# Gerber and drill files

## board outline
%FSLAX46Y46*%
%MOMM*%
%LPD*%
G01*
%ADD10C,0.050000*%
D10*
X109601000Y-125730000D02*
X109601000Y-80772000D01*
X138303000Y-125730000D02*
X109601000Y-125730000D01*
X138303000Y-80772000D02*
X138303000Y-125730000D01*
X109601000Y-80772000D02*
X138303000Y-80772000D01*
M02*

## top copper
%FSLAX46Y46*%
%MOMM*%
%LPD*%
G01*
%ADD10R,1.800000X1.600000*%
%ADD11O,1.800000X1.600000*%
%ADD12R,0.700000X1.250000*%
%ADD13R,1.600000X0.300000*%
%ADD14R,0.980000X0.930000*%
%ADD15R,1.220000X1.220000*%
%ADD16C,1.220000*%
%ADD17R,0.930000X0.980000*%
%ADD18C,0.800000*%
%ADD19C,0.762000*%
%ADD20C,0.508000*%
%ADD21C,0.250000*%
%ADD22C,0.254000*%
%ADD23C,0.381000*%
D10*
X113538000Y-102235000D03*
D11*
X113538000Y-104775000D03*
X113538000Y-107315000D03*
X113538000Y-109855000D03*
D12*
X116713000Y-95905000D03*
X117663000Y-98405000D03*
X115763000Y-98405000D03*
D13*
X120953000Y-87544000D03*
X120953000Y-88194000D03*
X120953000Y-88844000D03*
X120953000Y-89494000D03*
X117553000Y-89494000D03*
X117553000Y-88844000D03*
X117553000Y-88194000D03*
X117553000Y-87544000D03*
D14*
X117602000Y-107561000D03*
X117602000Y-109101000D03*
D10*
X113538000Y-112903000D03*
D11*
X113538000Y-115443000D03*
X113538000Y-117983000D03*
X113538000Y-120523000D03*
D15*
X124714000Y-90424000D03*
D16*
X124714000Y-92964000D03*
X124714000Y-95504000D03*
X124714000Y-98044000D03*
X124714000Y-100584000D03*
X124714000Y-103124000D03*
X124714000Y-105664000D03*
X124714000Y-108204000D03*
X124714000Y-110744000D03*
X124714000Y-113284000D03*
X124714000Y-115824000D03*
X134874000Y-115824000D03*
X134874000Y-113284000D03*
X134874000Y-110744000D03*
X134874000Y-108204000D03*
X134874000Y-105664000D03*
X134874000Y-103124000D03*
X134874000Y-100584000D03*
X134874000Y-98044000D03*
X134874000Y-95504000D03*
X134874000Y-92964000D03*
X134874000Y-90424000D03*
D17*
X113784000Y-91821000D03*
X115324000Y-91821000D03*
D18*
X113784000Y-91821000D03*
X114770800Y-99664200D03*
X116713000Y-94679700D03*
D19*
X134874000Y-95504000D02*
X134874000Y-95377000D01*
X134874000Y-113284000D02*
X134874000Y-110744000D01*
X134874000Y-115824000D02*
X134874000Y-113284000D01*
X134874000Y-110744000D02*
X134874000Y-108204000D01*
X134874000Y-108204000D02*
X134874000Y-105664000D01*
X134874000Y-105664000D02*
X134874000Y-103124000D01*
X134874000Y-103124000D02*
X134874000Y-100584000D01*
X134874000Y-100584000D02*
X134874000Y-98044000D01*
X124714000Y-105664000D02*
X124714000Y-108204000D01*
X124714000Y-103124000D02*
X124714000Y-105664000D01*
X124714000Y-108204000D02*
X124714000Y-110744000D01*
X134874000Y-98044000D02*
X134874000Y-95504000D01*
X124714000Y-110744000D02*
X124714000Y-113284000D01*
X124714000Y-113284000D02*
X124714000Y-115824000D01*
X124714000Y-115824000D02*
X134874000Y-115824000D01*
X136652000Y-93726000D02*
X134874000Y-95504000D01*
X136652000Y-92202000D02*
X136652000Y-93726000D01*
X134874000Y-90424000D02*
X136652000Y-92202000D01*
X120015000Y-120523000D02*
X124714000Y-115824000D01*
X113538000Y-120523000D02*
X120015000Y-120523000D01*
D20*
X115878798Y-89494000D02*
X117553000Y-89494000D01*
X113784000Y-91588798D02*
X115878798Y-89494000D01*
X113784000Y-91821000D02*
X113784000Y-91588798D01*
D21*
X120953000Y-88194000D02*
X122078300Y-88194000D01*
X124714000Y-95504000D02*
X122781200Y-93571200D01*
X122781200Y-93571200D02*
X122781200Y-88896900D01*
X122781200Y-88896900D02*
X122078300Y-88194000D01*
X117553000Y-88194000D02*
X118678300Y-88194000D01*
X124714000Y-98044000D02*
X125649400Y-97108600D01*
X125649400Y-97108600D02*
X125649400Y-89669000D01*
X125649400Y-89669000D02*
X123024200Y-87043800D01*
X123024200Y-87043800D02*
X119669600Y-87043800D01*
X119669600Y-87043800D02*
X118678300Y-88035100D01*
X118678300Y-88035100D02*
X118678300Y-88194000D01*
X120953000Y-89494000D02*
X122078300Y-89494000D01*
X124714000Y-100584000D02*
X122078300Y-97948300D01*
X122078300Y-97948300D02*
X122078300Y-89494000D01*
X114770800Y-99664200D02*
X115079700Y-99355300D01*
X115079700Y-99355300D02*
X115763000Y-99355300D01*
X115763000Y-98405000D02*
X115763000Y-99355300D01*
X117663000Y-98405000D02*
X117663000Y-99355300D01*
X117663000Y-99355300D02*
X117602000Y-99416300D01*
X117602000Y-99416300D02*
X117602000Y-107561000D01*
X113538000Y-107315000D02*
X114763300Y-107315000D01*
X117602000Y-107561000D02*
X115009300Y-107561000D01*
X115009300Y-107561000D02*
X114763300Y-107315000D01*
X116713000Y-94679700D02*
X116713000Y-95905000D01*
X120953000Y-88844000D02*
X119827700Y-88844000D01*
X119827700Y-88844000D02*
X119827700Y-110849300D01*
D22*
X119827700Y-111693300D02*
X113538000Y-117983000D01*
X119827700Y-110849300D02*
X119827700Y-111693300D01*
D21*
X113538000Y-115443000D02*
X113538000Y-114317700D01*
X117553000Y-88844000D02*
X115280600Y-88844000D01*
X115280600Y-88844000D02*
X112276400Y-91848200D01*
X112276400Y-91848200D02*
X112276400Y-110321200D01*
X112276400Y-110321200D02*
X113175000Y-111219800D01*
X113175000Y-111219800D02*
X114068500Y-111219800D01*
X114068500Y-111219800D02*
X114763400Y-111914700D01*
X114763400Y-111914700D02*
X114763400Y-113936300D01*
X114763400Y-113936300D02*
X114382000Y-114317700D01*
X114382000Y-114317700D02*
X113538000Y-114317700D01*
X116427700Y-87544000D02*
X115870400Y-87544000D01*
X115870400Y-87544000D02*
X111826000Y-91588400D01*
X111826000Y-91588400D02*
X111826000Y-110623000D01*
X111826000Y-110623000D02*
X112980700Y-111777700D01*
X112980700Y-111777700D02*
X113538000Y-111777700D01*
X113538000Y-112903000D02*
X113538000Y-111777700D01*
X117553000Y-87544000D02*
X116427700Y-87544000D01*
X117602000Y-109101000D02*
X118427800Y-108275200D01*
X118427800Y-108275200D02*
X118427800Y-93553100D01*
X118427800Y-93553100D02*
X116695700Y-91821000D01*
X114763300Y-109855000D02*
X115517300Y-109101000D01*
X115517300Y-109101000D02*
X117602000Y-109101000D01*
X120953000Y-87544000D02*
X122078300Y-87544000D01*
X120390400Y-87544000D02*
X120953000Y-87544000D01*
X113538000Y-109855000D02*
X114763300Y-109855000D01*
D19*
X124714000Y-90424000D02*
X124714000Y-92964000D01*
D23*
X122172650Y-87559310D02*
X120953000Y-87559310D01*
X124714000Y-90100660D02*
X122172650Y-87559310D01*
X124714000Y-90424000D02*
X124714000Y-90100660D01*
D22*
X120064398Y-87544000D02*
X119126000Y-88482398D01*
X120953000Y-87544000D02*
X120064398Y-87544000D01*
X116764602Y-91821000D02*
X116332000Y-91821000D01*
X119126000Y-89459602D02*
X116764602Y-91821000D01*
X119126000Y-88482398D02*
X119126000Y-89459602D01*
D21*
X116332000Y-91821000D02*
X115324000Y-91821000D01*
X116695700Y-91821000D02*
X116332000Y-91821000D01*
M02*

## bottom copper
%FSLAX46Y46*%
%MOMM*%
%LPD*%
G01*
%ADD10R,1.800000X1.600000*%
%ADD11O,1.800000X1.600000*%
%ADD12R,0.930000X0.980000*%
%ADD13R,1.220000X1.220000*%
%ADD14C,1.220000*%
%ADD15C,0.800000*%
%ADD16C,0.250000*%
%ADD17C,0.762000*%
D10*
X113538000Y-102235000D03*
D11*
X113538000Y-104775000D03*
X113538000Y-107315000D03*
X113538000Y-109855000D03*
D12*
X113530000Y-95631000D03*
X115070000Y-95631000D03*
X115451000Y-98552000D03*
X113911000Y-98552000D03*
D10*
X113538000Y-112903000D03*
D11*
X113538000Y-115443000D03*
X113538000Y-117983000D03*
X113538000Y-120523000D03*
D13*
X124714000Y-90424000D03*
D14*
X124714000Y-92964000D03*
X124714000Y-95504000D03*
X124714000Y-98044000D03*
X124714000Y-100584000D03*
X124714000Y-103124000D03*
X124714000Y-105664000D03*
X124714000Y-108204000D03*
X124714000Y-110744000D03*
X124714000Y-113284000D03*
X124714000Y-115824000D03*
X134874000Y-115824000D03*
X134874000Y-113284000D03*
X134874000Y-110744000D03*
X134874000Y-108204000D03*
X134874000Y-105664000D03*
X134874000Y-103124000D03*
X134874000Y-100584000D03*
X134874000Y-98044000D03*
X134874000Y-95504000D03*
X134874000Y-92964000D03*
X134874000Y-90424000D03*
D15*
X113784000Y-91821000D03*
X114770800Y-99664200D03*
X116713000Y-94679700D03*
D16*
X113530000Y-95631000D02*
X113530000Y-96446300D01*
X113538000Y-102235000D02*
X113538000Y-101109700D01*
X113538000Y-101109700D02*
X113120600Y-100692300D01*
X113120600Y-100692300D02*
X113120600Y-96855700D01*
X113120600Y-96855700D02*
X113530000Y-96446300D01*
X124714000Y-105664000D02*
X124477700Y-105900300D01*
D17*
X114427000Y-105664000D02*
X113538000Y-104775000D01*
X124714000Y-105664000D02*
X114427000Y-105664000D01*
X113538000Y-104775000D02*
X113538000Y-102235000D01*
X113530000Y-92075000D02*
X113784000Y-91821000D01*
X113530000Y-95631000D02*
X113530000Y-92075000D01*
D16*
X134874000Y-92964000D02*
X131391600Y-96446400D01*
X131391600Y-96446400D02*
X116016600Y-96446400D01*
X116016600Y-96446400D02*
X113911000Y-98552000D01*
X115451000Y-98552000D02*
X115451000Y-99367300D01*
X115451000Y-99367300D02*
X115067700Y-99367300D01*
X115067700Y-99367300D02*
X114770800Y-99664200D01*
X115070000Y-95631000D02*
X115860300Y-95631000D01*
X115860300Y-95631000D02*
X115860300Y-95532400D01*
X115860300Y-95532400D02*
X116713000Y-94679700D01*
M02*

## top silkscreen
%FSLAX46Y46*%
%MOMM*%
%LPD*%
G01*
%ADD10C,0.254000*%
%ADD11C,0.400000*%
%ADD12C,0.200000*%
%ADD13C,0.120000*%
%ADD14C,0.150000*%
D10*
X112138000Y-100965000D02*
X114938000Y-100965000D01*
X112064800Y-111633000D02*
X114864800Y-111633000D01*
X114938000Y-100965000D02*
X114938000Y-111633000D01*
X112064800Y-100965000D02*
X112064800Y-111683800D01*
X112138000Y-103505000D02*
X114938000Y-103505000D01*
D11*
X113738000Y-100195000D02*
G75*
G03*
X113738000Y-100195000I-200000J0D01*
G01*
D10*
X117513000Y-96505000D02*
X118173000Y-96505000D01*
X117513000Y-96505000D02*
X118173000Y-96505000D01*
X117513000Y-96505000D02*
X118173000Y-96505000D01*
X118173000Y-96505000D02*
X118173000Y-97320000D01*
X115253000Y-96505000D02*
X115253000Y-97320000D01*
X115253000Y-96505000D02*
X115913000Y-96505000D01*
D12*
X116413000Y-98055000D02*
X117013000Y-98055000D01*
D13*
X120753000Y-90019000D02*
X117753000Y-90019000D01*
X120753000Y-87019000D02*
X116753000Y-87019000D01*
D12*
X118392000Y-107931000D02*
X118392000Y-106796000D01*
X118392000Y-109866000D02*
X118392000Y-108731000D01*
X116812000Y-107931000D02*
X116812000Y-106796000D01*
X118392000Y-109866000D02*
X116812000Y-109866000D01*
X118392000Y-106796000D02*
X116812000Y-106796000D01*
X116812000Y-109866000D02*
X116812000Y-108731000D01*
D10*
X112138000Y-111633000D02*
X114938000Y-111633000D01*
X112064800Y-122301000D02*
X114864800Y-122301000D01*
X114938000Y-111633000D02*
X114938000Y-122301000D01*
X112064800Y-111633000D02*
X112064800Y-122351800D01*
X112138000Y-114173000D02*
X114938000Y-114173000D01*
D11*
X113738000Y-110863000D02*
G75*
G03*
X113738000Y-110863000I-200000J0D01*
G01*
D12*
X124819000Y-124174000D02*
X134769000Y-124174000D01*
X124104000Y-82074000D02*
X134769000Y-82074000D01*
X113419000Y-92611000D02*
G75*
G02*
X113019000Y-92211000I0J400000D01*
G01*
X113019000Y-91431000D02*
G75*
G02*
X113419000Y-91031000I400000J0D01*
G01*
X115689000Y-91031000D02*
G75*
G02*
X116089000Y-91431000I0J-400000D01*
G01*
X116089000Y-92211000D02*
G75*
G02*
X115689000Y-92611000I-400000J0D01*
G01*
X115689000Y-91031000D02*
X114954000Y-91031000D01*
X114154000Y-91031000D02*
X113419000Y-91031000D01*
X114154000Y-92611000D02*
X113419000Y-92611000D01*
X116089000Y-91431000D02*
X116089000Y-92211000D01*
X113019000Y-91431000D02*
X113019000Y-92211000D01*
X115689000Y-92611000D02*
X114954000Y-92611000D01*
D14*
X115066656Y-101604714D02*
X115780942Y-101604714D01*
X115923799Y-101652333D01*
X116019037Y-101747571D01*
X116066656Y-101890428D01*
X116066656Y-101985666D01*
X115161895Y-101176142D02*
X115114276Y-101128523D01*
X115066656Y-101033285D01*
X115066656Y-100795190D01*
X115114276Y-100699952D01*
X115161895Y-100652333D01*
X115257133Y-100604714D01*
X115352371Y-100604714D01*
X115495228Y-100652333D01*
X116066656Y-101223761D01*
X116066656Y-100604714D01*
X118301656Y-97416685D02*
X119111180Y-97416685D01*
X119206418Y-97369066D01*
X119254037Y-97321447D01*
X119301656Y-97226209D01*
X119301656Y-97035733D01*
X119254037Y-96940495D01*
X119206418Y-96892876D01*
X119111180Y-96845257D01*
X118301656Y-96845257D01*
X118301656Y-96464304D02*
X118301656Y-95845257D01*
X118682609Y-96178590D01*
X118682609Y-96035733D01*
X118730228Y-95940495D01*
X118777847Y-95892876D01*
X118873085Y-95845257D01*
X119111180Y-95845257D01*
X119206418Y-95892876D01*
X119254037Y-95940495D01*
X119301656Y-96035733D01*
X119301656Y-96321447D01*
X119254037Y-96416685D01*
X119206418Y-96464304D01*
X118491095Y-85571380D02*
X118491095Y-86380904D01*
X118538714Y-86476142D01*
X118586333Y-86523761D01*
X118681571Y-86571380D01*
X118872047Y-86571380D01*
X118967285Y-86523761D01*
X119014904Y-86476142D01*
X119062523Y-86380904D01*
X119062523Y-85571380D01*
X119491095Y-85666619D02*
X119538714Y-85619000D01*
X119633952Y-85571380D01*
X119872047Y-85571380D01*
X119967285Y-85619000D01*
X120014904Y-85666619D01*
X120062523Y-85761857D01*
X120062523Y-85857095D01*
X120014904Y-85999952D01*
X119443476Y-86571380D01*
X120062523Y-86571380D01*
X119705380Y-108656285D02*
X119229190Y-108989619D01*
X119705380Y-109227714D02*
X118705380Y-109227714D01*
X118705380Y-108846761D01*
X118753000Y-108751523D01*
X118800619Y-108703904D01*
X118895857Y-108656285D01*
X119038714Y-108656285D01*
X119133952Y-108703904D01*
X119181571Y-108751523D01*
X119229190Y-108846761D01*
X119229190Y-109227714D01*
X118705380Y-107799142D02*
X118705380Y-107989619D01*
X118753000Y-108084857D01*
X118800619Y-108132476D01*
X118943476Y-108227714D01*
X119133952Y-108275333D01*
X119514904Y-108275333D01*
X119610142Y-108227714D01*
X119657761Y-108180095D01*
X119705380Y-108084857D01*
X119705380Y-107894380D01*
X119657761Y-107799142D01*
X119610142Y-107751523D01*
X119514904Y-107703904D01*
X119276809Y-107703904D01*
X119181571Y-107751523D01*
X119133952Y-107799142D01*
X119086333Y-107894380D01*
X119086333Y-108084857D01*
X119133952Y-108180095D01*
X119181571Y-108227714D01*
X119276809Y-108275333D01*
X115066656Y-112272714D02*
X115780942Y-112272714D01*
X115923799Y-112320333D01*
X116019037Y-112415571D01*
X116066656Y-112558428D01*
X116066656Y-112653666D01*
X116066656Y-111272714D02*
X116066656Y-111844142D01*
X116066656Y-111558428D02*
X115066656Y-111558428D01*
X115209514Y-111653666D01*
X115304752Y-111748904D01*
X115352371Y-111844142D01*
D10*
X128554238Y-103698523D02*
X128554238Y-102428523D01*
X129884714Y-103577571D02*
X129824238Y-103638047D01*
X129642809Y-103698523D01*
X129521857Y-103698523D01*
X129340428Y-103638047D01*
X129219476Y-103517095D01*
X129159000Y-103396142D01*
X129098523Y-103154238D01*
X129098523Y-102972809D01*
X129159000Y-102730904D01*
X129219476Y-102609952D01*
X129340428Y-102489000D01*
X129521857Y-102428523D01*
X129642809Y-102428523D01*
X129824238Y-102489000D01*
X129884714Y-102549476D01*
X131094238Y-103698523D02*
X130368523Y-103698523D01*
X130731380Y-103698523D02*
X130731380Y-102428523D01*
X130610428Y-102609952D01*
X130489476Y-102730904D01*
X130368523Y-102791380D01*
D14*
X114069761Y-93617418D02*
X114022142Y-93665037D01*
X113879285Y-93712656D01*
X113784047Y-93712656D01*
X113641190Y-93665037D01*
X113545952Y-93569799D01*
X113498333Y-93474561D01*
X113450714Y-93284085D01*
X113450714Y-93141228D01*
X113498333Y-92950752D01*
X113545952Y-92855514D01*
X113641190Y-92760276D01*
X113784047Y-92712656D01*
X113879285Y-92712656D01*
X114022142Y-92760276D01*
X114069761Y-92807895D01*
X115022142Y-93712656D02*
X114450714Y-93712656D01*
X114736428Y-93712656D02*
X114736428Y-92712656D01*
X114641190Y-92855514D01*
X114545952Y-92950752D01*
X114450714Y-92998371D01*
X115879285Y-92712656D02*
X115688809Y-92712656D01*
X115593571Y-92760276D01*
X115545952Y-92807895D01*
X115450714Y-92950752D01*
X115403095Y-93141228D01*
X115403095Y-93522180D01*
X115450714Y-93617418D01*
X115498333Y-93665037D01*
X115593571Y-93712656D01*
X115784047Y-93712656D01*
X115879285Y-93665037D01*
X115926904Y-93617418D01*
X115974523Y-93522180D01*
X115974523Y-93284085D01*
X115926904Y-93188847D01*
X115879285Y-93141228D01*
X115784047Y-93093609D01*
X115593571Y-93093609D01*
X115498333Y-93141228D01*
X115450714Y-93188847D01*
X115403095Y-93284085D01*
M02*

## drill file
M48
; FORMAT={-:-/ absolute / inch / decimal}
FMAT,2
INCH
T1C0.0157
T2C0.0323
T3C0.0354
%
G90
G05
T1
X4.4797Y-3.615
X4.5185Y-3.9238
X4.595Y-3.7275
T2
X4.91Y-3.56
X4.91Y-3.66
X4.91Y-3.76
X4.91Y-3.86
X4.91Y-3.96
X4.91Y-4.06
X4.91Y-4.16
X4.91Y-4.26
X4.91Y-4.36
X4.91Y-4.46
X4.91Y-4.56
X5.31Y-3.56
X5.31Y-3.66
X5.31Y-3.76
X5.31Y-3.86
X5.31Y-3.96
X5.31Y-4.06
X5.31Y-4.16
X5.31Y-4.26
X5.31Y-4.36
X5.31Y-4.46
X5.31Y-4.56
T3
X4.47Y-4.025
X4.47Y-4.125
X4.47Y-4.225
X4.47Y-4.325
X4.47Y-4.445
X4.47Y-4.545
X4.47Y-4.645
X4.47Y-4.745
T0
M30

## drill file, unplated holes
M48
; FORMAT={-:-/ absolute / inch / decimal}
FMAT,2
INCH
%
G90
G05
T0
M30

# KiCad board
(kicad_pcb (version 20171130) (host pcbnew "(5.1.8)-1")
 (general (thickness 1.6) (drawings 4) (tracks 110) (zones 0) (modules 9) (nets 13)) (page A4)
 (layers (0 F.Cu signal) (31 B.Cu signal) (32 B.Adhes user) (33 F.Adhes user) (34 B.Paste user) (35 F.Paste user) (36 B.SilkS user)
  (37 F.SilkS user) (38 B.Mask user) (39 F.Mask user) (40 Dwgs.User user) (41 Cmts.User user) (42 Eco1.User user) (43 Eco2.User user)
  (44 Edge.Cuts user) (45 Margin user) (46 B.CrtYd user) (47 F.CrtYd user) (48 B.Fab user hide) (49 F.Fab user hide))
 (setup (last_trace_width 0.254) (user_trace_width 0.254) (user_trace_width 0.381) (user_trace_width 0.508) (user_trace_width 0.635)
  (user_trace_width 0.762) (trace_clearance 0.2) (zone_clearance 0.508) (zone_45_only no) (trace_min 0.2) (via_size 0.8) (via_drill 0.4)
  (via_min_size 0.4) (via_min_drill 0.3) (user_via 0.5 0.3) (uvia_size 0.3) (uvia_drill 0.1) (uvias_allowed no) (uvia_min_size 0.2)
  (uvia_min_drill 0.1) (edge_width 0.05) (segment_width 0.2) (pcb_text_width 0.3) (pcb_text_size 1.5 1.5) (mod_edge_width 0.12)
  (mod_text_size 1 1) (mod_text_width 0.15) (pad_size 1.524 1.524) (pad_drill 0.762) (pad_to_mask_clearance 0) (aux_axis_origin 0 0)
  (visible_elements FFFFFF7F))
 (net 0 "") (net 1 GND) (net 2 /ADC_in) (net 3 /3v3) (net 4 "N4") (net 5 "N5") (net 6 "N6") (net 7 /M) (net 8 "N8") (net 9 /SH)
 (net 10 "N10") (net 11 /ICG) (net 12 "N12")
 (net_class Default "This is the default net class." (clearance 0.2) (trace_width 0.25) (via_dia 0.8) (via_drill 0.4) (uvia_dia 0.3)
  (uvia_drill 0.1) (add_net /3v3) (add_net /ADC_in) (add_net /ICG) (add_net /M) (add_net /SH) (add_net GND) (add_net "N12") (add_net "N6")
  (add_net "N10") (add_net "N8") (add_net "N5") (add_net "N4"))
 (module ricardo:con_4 (layer F.Cu) (at 113.538 111.125 270)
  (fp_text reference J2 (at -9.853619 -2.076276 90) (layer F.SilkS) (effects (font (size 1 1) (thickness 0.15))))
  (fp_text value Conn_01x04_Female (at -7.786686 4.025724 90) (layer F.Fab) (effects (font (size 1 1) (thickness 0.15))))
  (fp_line (start -10.16 1.4) (end -10.16 -1.4) (layer F.SilkS) (width 0.254))
  (fp_line (start 0.508 1.4732) (end 0.508 -1.3268) (layer F.SilkS) (width 0.254))
  (fp_line (start -10.16 -1.4) (end 0.508 -1.4) (layer F.SilkS) (width 0.254))
  (fp_line (start -10.16 1.4732) (end 0.5588 1.4732) (layer F.SilkS) (width 0.254))
  (fp_line (start -7.62 1.4) (end -7.62 -1.4) (layer F.SilkS) (width 0.254))
  (fp_circle (center -10.93 0) (end -10.73 0) (layer F.SilkS) (width 0.4))
  (pad 1 thru_hole rect (at -8.89 0 270) (size 1.6 1.8) (drill 0.9) (layers *.Cu *.Mask) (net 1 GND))
  (pad 2 thru_hole oval (at -6.35 0 270) (size 1.6 1.8) (drill 0.9) (layers *.Cu *.Mask) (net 1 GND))
  (pad 3 thru_hole oval (at -3.81 0 270) (size 1.6 1.8) (drill 0.9) (layers *.Cu *.Mask) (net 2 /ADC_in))
  (pad 4 thru_hole oval (at -1.27 0 270) (size 1.6 1.8) (drill 0.9) (layers *.Cu *.Mask) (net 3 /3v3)))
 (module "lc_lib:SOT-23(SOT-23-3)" (layer F.Cu) (at 116.713 97.155 270)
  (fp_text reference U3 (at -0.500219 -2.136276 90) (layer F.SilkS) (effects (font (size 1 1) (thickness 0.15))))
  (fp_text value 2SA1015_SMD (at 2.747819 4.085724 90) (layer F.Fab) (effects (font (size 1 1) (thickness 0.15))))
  (fp_line (start -0.65 -0.8) (end -0.65 -1.46) (layer F.SilkS) (width 0.254))
  (fp_line (start -0.65 -0.8) (end -0.65 -1.46) (layer F.SilkS) (width 0.254))
  (fp_line (start -0.65 -0.8) (end -0.65 -1.46) (layer F.SilkS) (width 0.254))
  (fp_line (start -0.65 -1.46) (end 0.165 -1.46) (layer F.SilkS) (width 0.254))
  (fp_line (start -0.65 1.46) (end 0.165 1.46) (layer F.SilkS) (width 0.254))
  (fp_line (start -0.65 1.46) (end -0.65 0.8) (layer F.SilkS) (width 0.254))
  (fp_line (start 0.9 0.3) (end 0.9 -0.3) (layer F.SilkS) (width 0.2))
  (pad 3 smd rect (at -1.25 0 180) (size 0.7 1.25) (layers F.Cu F.Paste F.Mask) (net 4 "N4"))
  (pad 2 smd rect (at 1.25 -0.95 180) (size 0.7 1.25) (layers F.Cu F.Paste F.Mask) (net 2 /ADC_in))
  (pad 1 smd rect (at 1.25 0.95 180) (size 0.7 1.25) (layers F.Cu F.Paste F.Mask) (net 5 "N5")))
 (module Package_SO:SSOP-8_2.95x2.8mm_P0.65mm (layer F.Cu) (at 119.253 88.519)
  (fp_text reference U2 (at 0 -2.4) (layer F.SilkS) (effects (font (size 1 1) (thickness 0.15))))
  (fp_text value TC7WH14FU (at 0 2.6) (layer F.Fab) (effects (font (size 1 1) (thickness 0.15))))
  (fp_line (start 1.5 1.5) (end -1.5 1.5) (layer F.SilkS) (width 0.12))
  (fp_line (start 1.5 -1.5) (end -2.5 -1.5) (layer F.SilkS) (width 0.12))
  (pad 8 smd rect (at 1.7 -0.975 270) (size 0.3 1.6) (layers F.Cu F.Paste F.Mask) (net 3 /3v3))
  (pad 7 smd rect (at 1.7 -0.325 270) (size 0.3 1.6) (layers F.Cu F.Paste F.Mask) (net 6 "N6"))
  (pad 6 smd rect (at 1.7 0.325 270) (size 0.3 1.6) (layers F.Cu F.Paste F.Mask) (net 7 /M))
  (pad 5 smd rect (at 1.7 0.975 270) (size 0.3 1.6) (layers F.Cu F.Paste F.Mask) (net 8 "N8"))
  (pad 4 smd rect (at -1.7 0.975 270) (size 0.3 1.6) (layers F.Cu F.Paste F.Mask) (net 1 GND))
  (pad 3 smd rect (at -1.7 0.325 270) (size 0.3 1.6) (layers F.Cu F.Paste F.Mask) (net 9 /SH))
  (pad 2 smd rect (at -1.7 -0.325 270) (size 0.3 1.6) (layers F.Cu F.Paste F.Mask) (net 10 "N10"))
  (pad 1 smd rect (at -1.7 -0.975 270) (size 0.3 1.6) (layers F.Cu F.Paste F.Mask) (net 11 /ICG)))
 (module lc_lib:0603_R (layer B.Cu) (at 114.3 95.631 180)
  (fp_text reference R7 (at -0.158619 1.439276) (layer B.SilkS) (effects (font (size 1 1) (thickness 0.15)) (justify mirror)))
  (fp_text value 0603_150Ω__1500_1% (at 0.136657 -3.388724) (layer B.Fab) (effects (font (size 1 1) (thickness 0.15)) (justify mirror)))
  (pad 2 smd rect (at 0.77 0 180) (size 0.93 0.98) (layers B.Cu B.Paste B.Mask) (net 1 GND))
  (pad 1 smd rect (at -0.77 0 180) (size 0.93 0.98) (layers B.Cu B.Paste B.Mask) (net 4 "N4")))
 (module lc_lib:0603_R (layer F.Cu) (at 117.602 108.331 90)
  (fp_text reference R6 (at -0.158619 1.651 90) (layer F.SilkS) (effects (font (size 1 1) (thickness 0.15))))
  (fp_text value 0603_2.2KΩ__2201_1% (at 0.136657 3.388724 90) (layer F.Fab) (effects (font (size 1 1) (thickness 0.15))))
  (fp_line (start 0.4 0.79) (end 1.535 0.79) (layer F.SilkS) (width 0.2))
  (fp_line (start -1.535 0.79) (end -0.4 0.79) (layer F.SilkS) (width 0.2))
  (fp_line (start 0.4 -0.79) (end 1.535 -0.79) (layer F.SilkS) (width 0.2))
  (fp_line (start -1.535 0.79) (end -1.535 -0.79) (layer F.SilkS) (width 0.2))
  (fp_line (start 1.535 0.79) (end 1.535 -0.79) (layer F.SilkS) (width 0.2))
  (fp_line (start -1.535 -0.79) (end -0.4 -0.79) (layer F.SilkS) (width 0.2))
  (pad 2 smd rect (at 0.77 0 90) (size 0.93 0.98) (layers F.Cu F.Paste F.Mask) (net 2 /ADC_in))
  (pad 1 smd rect (at -0.77 0 90) (size 0.93 0.98) (layers F.Cu F.Paste F.Mask) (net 3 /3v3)))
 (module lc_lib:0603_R (layer B.Cu) (at 114.681 98.552)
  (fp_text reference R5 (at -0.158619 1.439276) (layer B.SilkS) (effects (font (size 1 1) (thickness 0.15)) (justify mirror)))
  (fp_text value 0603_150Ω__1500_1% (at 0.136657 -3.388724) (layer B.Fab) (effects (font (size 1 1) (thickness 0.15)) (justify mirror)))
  (pad 2 smd rect (at 0.77 0) (size 0.93 0.98) (layers B.Cu B.Paste B.Mask) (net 5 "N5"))
  (pad 1 smd rect (at -0.77 0) (size 0.93 0.98) (layers B.Cu B.Paste B.Mask) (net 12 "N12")))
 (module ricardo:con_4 (layer F.Cu) (at 113.538 121.793 270)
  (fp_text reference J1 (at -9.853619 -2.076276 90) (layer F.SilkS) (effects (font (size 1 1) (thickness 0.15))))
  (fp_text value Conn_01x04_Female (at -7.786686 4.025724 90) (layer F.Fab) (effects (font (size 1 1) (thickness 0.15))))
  (fp_line (start -10.16 1.4) (end -10.16 -1.4) (layer F.SilkS) (width 0.254))
  (fp_line (start 0.508 1.4732) (end 0.508 -1.3268) (layer F.SilkS) (width 0.254))
  (fp_line (start -10.16 -1.4) (end 0.508 -1.4) (layer F.SilkS) (width 0.254))
  (fp_line (start -10.16 1.4732) (end 0.5588 1.4732) (layer F.SilkS) (width 0.254))
  (fp_line (start -7.62 1.4) (end -7.62 -1.4) (layer F.SilkS) (width 0.254))
  (fp_circle (center -10.93 0) (end -10.73 0) (layer F.SilkS) (width 0.4))
  (pad 1 thru_hole rect (at -8.89 0 270) (size 1.6 1.8) (drill 0.9) (layers *.Cu *.Mask) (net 11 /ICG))
  (pad 2 thru_hole oval (at -6.35 0 270) (size 1.6 1.8) (drill 0.9) (layers *.Cu *.Mask) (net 9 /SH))
  (pad 3 thru_hole oval (at -3.81 0 270) (size 1.6 1.8) (drill 0.9) (layers *.Cu *.Mask) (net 7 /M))
  (pad 4 thru_hole oval (at -1.27 0 270) (size 1.6 1.8) (drill 0.9) (layers *.Cu *.Mask) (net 1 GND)))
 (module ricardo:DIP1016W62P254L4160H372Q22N (layer F.Cu) (at 129.794 103.124)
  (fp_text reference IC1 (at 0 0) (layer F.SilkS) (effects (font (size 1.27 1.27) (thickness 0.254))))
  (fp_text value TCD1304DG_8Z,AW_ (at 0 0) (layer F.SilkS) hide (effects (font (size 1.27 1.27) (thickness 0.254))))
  (fp_line (start -4.975 21.05) (end 4.975 21.05) (layer F.SilkS) (width 0.2))
  (fp_line (start -5.69 -21.05) (end 4.975 -21.05) (layer F.SilkS) (width 0.2))
  (pad 1 thru_hole rect (at -5.08 -12.7) (size 1.22 1.22) (drill 0.82) (layers *.Cu *.Mask) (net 3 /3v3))
  (pad 2 thru_hole circle (at -5.08 -10.16) (size 1.22 1.22) (drill 0.82) (layers *.Cu *.Mask) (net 3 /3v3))
  (pad 3 thru_hole circle (at -5.08 -7.62) (size 1.22 1.22) (drill 0.82) (layers *.Cu *.Mask) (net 6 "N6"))
  (pad 4 thru_hole circle (at -5.08 -5.08) (size 1.22 1.22) (drill 0.82) (layers *.Cu *.Mask) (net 10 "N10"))
  (pad 5 thru_hole circle (at -5.08 -2.54) (size 1.22 1.22) (drill 0.82) (layers *.Cu *.Mask) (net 8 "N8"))
  (pad 6 thru_hole circle (at -5.08 0) (size 1.22 1.22) (drill 0.82) (layers *.Cu *.Mask) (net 1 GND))
  (pad 7 thru_hole circle (at -5.08 2.54) (size 1.22 1.22) (drill 0.82) (layers *.Cu *.Mask) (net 1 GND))
  (pad 8 thru_hole circle (at -5.08 5.08) (size 1.22 1.22) (drill 0.82) (layers *.Cu *.Mask) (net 1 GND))
  (pad 9 thru_hole circle (at -5.08 7.62) (size 1.22 1.22) (drill 0.82) (layers *.Cu *.Mask) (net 1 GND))
  (pad 10 thru_hole circle (at -5.08 10.16) (size 1.22 1.22) (drill 0.82) (layers *.Cu *.Mask) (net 1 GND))
  (pad 11 thru_hole circle (at -5.08 12.7) (size 1.22 1.22) (drill 0.82) (layers *.Cu *.Mask) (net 1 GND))
  (pad 12 thru_hole circle (at 5.08 12.7) (size 1.22 1.22) (drill 0.82) (layers *.Cu *.Mask) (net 1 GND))
  (pad 13 thru_hole circle (at 5.08 10.16) (size 1.22 1.22) (drill 0.82) (layers *.Cu *.Mask) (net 1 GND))
  (pad 14 thru_hole circle (at 5.08 7.62) (size 1.22 1.22) (drill 0.82) (layers *.Cu *.Mask) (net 1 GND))
  (pad 15 thru_hole circle (at 5.08 5.08) (size 1.22 1.22) (drill 0.82) (layers *.Cu *.Mask) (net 1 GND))
  (pad 16 thru_hole circle (at 5.08 2.54) (size 1.22 1.22) (drill 0.82) (layers *.Cu *.Mask) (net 1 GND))
  (pad 17 thru_hole circle (at 5.08 0) (size 1.22 1.22) (drill 0.82) (layers *.Cu *.Mask) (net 1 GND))
  (pad 18 thru_hole circle (at 5.08 -2.54) (size 1.22 1.22) (drill 0.82) (layers *.Cu *.Mask) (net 1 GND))
  (pad 19 thru_hole circle (at 5.08 -5.08) (size 1.22 1.22) (drill 0.82) (layers *.Cu *.Mask) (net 1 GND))
  (pad 20 thru_hole circle (at 5.08 -7.62) (size 1.22 1.22) (drill 0.82) (layers *.Cu *.Mask) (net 1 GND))
  (pad 21 thru_hole circle (at 5.08 -10.16) (size 1.22 1.22) (drill 0.82) (layers *.Cu *.Mask) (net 12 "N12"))
  (pad 22 thru_hole circle (at 5.08 -12.7) (size 1.22 1.22) (drill 0.82) (layers *.Cu *.Mask) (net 1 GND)))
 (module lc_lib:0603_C (layer F.Cu) (at 114.554 91.821 180)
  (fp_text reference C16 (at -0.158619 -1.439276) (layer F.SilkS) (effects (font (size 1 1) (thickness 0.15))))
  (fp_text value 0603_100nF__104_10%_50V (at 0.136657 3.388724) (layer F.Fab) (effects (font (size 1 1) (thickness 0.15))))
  (fp_arc (start 1.135 -0.39) (end 1.535 -0.39) (angle -90) (layer F.SilkS) (width 0.2))
  (fp_arc (start 1.135 0.39) (end 1.135 0.79) (angle -90) (layer F.SilkS) (width 0.2))
  (fp_arc (start -1.135 0.39) (end -1.535 0.39) (angle -90) (layer F.SilkS) (width 0.2))
  (fp_arc (start -1.135 -0.39) (end -1.135 -0.79) (angle -90) (layer F.SilkS) (width 0.2))
  (fp_line (start -1.135 0.79) (end -0.4 0.79) (layer F.SilkS) (width 0.2))
  (fp_line (start 0.4 0.79) (end 1.135 0.79) (layer F.SilkS) (width 0.2))
  (fp_line (start 0.4 -0.79) (end 1.135 -0.79) (layer F.SilkS) (width 0.2))
  (fp_line (start -1.535 0.39) (end -1.535 -0.39) (layer F.SilkS) (width 0.2))
  (fp_line (start 1.535 0.39) (end 1.535 -0.39) (layer F.SilkS) (width 0.2))
  (fp_line (start -1.135 -0.79) (end -0.4 -0.79) (layer F.SilkS) (width 0.2))
  (pad 2 smd rect (at 0.77 0 180) (size 0.93 0.98) (layers F.Cu F.Paste F.Mask) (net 1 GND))
  (pad 1 smd rect (at -0.77 0 180) (size 0.93 0.98) (layers F.Cu F.Paste F.Mask) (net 3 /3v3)))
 (gr_line (start 109.601 125.73) (end 109.601 80.772) (layer Edge.Cuts) (width 0.05))
 (gr_line (start 138.303 125.73) (end 109.601 125.73) (layer Edge.Cuts) (width 0.05))
 (gr_line (start 138.303 80.772) (end 138.303 125.73) (layer Edge.Cuts) (width 0.05))
 (gr_line (start 109.601 80.772) (end 138.303 80.772) (layer Edge.Cuts) (width 0.05))
 (segment (start 134.874 95.504) (end 134.874 95.377) (width 0.762) (layer F.Cu) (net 1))
 (segment (start 113.53 95.631) (end 113.53 96.4463) (width 0.25) (layer B.Cu) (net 1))
 (segment (start 113.538 102.235) (end 113.538 101.1097) (width 0.25) (layer B.Cu) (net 1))
 (segment (start 113.538 101.1097) (end 113.1206 100.6923) (width 0.25) (layer B.Cu) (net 1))
 (segment (start 113.1206 100.6923) (end 113.1206 96.8557) (width 0.25) (layer B.Cu) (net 1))
 (segment (start 113.1206 96.8557) (end 113.53 96.4463) (width 0.25) (layer B.Cu) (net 1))
 (segment (start 124.714 105.664) (end 124.4777 105.9003) (width 0.25) (layer B.Cu) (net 1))
 (segment (start 134.874 113.284) (end 134.874 110.744) (width 0.762) (layer F.Cu) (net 1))
 (segment (start 134.874 115.824) (end 134.874 113.284) (width 0.762) (layer F.Cu) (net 1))
 (segment (start 134.874 110.744) (end 134.874 108.204) (width 0.762) (layer F.Cu) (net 1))
 (segment (start 134.874 108.204) (end 134.874 105.664) (width 0.762) (layer F.Cu) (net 1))
 (segment (start 134.874 105.664) (end 134.874 103.124) (width 0.762) (layer F.Cu) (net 1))
 (segment (start 134.874 103.124) (end 134.874 100.584) (width 0.762) (layer F.Cu) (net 1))
 (segment (start 134.874 100.584) (end 134.874 98.044) (width 0.762) (layer F.Cu) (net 1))
 (segment (start 124.714 105.664) (end 124.714 108.204) (width 0.762) (layer F.Cu) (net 1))
 (segment (start 124.714 103.124) (end 124.714 105.664) (width 0.762) (layer F.Cu) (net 1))
 (segment (start 124.714 108.204) (end 124.714 110.744) (width 0.762) (layer F.Cu) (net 1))
 (segment (start 134.874 98.044) (end 134.874 95.504) (width 0.762) (layer F.Cu) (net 1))
 (segment (start 124.714 110.744) (end 124.714 113.284) (width 0.762) (layer F.Cu) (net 1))
 (segment (start 124.714 113.284) (end 124.714 115.824) (width 0.762) (layer F.Cu) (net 1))
 (segment (start 124.714 115.824) (end 134.874 115.824) (width 0.762) (layer F.Cu) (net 1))
 (segment (start 136.652 93.726) (end 134.874 95.504) (width 0.762) (layer F.Cu) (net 1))
 (segment (start 136.652 92.202) (end 136.652 93.726) (width 0.762) (layer F.Cu) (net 1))
 (segment (start 134.874 90.424) (end 136.652 92.202) (width 0.762) (layer F.Cu) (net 1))
 (segment (start 120.015 120.523) (end 124.714 115.824) (width 0.762) (layer F.Cu) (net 1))
 (segment (start 113.538 120.523) (end 120.015 120.523) (width 0.762) (layer F.Cu) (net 1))
 (segment (start 114.427 105.664) (end 113.538 104.775) (width 0.762) (layer B.Cu) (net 1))
 (segment (start 124.714 105.664) (end 114.427 105.664) (width 0.762) (layer B.Cu) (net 1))
 (segment (start 113.538 104.775) (end 113.538 102.235) (width 0.762) (layer B.Cu) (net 1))
 (via (at 113.784 91.821) (size 0.8) (drill 0.4) (layers F.Cu B.Cu) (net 1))
 (segment (start 113.53 92.075) (end 113.784 91.821) (width 0.762) (layer B.Cu) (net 1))
 (segment (start 113.53 95.631) (end 113.53 92.075) (width 0.762) (layer B.Cu) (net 1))
 (segment (start 115.878798 89.494) (end 117.553 89.494) (width 0.508) (layer F.Cu) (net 1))
 (segment (start 113.784 91.588798) (end 115.878798 89.494) (width 0.508) (layer F.Cu) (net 1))
 (segment (start 113.784 91.821) (end 113.784 91.588798) (width 0.508) (layer F.Cu) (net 1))
 (segment (start 120.953 88.194) (end 122.0783 88.194) (width 0.25) (layer F.Cu) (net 6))
 (segment (start 124.714 95.504) (end 122.7812 93.5712) (width 0.25) (layer F.Cu) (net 6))
 (segment (start 122.7812 93.5712) (end 122.7812 88.8969) (width 0.25) (layer F.Cu) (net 6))
 (segment (start 122.7812 88.8969) (end 122.0783 88.194) (width 0.25) (layer F.Cu) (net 6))
 (segment (start 117.553 88.194) (end 118.6783 88.194) (width 0.25) (layer F.Cu) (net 10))
 (segment (start 124.714 98.044) (end 125.6494 97.1086) (width 0.25) (layer F.Cu) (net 10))
 (segment (start 125.6494 97.1086) (end 125.6494 89.669) (width 0.25) (layer F.Cu) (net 10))
 (segment (start 125.6494 89.669) (end 123.0242 87.0438) (width 0.25) (layer F.Cu) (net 10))
 (segment (start 123.0242 87.0438) (end 119.6696 87.0438) (width 0.25) (layer F.Cu) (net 10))
 (segment (start 119.6696 87.0438) (end 118.6783 88.0351) (width 0.25) (layer F.Cu) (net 10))
 (segment (start 118.6783 88.0351) (end 118.6783 88.194) (width 0.25) (layer F.Cu) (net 10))
 (segment (start 120.953 89.494) (end 122.0783 89.494) (width 0.25) (layer F.Cu) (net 8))
 (segment (start 124.714 100.584) (end 122.0783 97.9483) (width 0.25) (layer F.Cu) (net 8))
 (segment (start 122.0783 97.9483) (end 122.0783 89.494) (width 0.25) (layer F.Cu) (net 8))
 (segment (start 134.874 92.964) (end 131.3916 96.4464) (width 0.25) (layer B.Cu) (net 12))
 (segment (start 131.3916 96.4464) (end 116.0166 96.4464) (width 0.25) (layer B.Cu) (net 12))
 (segment (start 116.0166 96.4464) (end 113.911 98.552) (width 0.25) (layer B.Cu) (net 12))
 (segment (start 115.451 98.552) (end 115.451 99.3673) (width 0.25) (layer B.Cu) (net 5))
 (segment (start 114.7708 99.6642) (end 115.0797 99.3553) (width 0.25) (layer F.Cu) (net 5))
 (segment (start 115.0797 99.3553) (end 115.763 99.3553) (width 0.25) (layer F.Cu) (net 5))
 (segment (start 115.451 99.3673) (end 115.0677 99.3673) (width 0.25) (layer B.Cu) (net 5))
 (segment (start 115.0677 99.3673) (end 114.7708 99.6642) (width 0.25) (layer B.Cu) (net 5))
 (segment (start 115.763 98.405) (end 115.763 99.3553) (width 0.25) (layer F.Cu) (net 5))
 (via (at 114.7708 99.6642) (size 0.8) (layers F.Cu B.Cu) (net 5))
 (segment (start 117.663 98.405) (end 117.663 99.3553) (width 0.25) (layer F.Cu) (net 2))
 (segment (start 117.663 99.3553) (end 117.602 99.4163) (width 0.25) (layer F.Cu) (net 2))
 (segment (start 117.602 99.4163) (end 117.602 107.561) (width 0.25) (layer F.Cu) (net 2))
 (segment (start 113.538 107.315) (end 114.7633 107.315) (width 0.25) (layer F.Cu) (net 2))
 (segment (start 117.602 107.561) (end 115.0093 107.561) (width 0.25) (layer F.Cu) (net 2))
 (segment (start 115.0093 107.561) (end 114.7633 107.315) (width 0.25) (layer F.Cu) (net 2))
 (segment (start 115.07 95.631) (end 115.8603 95.631) (width 0.25) (layer B.Cu) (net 4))
 (segment (start 116.713 94.6797) (end 116.713 95.905) (width 0.25) (layer F.Cu) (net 4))
 (segment (start 115.8603 95.631) (end 115.8603 95.5324) (width 0.25) (layer B.Cu) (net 4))
 (segment (start 115.8603 95.5324) (end 116.713 94.6797) (width 0.25) (layer B.Cu) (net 4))
 (via (at 116.713 94.6797) (size 0.8) (layers F.Cu B.Cu) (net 4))
 (segment (start 120.953 88.844) (end 119.8277 88.844) (width 0.25) (layer F.Cu) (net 7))
 (segment (start 119.8277 88.844) (end 119.8277 110.8493) (width 0.25) (layer F.Cu) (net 7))
 (segment (start 119.8277 111.6933) (end 113.538 117.983) (width 0.254) (layer F.Cu) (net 7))
 (segment (start 119.8277 110.8493) (end 119.8277 111.6933) (width 0.254) (layer F.Cu) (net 7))
 (segment (start 113.538 115.443) (end 113.538 114.3177) (width 0.25) (layer F.Cu) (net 9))
 (segment (start 117.553 88.844) (end 115.2806 88.844) (width 0.25) (layer F.Cu) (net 9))
 (segment (start 115.2806 88.844) (end 112.2764 91.8482) (width 0.25) (layer F.Cu) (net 9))
 (segment (start 112.2764 91.8482) (end 112.2764 110.3212) (width 0.25) (layer F.Cu) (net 9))
 (segment (start 112.2764 110.3212) (end 113.175 111.2198) (width 0.25) (layer F.Cu) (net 9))
 (segment (start 113.175 111.2198) (end 114.0685 111.2198) (width 0.25) (layer F.Cu) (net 9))
 (segment (start 114.0685 111.2198) (end 114.7634 111.9147) (width 0.25) (layer F.Cu) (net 9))
 (segment (start 114.7634 111.9147) (end 114.7634 113.9363) (width 0.25) (layer F.Cu) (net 9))
 (segment (start 114.7634 113.9363) (end 114.382 114.3177) (width 0.25) (layer F.Cu) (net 9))
 (segment (start 114.382 114.3177) (end 113.538 114.3177) (width 0.25) (layer F.Cu) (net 9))
 (segment (start 116.4277 87.544) (end 115.8704 87.544) (width 0.25) (layer F.Cu) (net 11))
 (segment (start 115.8704 87.544) (end 111.826 91.5884) (width 0.25) (layer F.Cu) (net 11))
 (segment (start 111.826 91.5884) (end 111.826 110.623) (width 0.25) (layer F.Cu) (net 11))
 (segment (start 111.826 110.623) (end 112.9807 111.7777) (width 0.25) (layer F.Cu) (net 11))
 (segment (start 112.9807 111.7777) (end 113.538 111.7777) (width 0.25) (layer F.Cu) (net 11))
 (segment (start 113.538 112.903) (end 113.538 111.7777) (width 0.25) (layer F.Cu) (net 11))
 (segment (start 117.553 87.544) (end 116.4277 87.544) (width 0.25) (layer F.Cu) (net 11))
 (segment (start 117.602 109.101) (end 118.4278 108.2752) (width 0.25) (layer F.Cu) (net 3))
 (segment (start 118.4278 108.2752) (end 118.4278 93.5531) (width 0.25) (layer F.Cu) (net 3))
 (segment (start 118.4278 93.5531) (end 116.6957 91.821) (width 0.25) (layer F.Cu) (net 3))
 (segment (start 114.7633 109.855) (end 115.5173 109.101) (width 0.25) (layer F.Cu) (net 3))
 (segment (start 115.5173 109.101) (end 117.602 109.101) (width 0.25) (layer F.Cu) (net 3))
 (segment (start 120.953 87.544) (end 122.0783 87.544) (width 0.25) (layer F.Cu) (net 3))
 (segment (start 120.3904 87.544) (end 120.953 87.544) (width 0.25) (layer F.Cu) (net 3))
 (segment (start 113.538 109.855) (end 114.7633 109.855) (width 0.25) (layer F.Cu) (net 3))
 (segment (start 124.714 90.424) (end 124.714 92.964) (width 0.762) (layer F.Cu) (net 3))
 (segment (start 122.17265 87.55931) (end 120.953 87.55931) (width 0.381) (layer F.Cu) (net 3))
 (segment (start 124.714 90.10066) (end 122.17265 87.55931) (width 0.381) (layer F.Cu) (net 3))
 (segment (start 124.714 90.424) (end 124.714 90.10066) (width 0.381) (layer F.Cu) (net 3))
 (segment (start 120.064398 87.544) (end 119.126 88.482398) (width 0.254) (layer F.Cu) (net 3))
 (segment (start 120.953 87.544) (end 120.064398 87.544) (width 0.254) (layer F.Cu) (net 3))
 (segment (start 116.764602 91.821) (end 116.332 91.821) (width 0.254) (layer F.Cu) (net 3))
 (segment (start 119.126 89.459602) (end 116.764602 91.821) (width 0.254) (layer F.Cu) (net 3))
 (segment (start 119.126 88.482398) (end 119.126 89.459602) (width 0.254) (layer F.Cu) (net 3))
 (segment (start 116.332 91.821) (end 115.324 91.821) (width 0.25) (layer F.Cu) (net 3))
 (segment (start 116.6957 91.821) (end 116.332 91.821) (width 0.25) (layer F.Cu) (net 3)))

